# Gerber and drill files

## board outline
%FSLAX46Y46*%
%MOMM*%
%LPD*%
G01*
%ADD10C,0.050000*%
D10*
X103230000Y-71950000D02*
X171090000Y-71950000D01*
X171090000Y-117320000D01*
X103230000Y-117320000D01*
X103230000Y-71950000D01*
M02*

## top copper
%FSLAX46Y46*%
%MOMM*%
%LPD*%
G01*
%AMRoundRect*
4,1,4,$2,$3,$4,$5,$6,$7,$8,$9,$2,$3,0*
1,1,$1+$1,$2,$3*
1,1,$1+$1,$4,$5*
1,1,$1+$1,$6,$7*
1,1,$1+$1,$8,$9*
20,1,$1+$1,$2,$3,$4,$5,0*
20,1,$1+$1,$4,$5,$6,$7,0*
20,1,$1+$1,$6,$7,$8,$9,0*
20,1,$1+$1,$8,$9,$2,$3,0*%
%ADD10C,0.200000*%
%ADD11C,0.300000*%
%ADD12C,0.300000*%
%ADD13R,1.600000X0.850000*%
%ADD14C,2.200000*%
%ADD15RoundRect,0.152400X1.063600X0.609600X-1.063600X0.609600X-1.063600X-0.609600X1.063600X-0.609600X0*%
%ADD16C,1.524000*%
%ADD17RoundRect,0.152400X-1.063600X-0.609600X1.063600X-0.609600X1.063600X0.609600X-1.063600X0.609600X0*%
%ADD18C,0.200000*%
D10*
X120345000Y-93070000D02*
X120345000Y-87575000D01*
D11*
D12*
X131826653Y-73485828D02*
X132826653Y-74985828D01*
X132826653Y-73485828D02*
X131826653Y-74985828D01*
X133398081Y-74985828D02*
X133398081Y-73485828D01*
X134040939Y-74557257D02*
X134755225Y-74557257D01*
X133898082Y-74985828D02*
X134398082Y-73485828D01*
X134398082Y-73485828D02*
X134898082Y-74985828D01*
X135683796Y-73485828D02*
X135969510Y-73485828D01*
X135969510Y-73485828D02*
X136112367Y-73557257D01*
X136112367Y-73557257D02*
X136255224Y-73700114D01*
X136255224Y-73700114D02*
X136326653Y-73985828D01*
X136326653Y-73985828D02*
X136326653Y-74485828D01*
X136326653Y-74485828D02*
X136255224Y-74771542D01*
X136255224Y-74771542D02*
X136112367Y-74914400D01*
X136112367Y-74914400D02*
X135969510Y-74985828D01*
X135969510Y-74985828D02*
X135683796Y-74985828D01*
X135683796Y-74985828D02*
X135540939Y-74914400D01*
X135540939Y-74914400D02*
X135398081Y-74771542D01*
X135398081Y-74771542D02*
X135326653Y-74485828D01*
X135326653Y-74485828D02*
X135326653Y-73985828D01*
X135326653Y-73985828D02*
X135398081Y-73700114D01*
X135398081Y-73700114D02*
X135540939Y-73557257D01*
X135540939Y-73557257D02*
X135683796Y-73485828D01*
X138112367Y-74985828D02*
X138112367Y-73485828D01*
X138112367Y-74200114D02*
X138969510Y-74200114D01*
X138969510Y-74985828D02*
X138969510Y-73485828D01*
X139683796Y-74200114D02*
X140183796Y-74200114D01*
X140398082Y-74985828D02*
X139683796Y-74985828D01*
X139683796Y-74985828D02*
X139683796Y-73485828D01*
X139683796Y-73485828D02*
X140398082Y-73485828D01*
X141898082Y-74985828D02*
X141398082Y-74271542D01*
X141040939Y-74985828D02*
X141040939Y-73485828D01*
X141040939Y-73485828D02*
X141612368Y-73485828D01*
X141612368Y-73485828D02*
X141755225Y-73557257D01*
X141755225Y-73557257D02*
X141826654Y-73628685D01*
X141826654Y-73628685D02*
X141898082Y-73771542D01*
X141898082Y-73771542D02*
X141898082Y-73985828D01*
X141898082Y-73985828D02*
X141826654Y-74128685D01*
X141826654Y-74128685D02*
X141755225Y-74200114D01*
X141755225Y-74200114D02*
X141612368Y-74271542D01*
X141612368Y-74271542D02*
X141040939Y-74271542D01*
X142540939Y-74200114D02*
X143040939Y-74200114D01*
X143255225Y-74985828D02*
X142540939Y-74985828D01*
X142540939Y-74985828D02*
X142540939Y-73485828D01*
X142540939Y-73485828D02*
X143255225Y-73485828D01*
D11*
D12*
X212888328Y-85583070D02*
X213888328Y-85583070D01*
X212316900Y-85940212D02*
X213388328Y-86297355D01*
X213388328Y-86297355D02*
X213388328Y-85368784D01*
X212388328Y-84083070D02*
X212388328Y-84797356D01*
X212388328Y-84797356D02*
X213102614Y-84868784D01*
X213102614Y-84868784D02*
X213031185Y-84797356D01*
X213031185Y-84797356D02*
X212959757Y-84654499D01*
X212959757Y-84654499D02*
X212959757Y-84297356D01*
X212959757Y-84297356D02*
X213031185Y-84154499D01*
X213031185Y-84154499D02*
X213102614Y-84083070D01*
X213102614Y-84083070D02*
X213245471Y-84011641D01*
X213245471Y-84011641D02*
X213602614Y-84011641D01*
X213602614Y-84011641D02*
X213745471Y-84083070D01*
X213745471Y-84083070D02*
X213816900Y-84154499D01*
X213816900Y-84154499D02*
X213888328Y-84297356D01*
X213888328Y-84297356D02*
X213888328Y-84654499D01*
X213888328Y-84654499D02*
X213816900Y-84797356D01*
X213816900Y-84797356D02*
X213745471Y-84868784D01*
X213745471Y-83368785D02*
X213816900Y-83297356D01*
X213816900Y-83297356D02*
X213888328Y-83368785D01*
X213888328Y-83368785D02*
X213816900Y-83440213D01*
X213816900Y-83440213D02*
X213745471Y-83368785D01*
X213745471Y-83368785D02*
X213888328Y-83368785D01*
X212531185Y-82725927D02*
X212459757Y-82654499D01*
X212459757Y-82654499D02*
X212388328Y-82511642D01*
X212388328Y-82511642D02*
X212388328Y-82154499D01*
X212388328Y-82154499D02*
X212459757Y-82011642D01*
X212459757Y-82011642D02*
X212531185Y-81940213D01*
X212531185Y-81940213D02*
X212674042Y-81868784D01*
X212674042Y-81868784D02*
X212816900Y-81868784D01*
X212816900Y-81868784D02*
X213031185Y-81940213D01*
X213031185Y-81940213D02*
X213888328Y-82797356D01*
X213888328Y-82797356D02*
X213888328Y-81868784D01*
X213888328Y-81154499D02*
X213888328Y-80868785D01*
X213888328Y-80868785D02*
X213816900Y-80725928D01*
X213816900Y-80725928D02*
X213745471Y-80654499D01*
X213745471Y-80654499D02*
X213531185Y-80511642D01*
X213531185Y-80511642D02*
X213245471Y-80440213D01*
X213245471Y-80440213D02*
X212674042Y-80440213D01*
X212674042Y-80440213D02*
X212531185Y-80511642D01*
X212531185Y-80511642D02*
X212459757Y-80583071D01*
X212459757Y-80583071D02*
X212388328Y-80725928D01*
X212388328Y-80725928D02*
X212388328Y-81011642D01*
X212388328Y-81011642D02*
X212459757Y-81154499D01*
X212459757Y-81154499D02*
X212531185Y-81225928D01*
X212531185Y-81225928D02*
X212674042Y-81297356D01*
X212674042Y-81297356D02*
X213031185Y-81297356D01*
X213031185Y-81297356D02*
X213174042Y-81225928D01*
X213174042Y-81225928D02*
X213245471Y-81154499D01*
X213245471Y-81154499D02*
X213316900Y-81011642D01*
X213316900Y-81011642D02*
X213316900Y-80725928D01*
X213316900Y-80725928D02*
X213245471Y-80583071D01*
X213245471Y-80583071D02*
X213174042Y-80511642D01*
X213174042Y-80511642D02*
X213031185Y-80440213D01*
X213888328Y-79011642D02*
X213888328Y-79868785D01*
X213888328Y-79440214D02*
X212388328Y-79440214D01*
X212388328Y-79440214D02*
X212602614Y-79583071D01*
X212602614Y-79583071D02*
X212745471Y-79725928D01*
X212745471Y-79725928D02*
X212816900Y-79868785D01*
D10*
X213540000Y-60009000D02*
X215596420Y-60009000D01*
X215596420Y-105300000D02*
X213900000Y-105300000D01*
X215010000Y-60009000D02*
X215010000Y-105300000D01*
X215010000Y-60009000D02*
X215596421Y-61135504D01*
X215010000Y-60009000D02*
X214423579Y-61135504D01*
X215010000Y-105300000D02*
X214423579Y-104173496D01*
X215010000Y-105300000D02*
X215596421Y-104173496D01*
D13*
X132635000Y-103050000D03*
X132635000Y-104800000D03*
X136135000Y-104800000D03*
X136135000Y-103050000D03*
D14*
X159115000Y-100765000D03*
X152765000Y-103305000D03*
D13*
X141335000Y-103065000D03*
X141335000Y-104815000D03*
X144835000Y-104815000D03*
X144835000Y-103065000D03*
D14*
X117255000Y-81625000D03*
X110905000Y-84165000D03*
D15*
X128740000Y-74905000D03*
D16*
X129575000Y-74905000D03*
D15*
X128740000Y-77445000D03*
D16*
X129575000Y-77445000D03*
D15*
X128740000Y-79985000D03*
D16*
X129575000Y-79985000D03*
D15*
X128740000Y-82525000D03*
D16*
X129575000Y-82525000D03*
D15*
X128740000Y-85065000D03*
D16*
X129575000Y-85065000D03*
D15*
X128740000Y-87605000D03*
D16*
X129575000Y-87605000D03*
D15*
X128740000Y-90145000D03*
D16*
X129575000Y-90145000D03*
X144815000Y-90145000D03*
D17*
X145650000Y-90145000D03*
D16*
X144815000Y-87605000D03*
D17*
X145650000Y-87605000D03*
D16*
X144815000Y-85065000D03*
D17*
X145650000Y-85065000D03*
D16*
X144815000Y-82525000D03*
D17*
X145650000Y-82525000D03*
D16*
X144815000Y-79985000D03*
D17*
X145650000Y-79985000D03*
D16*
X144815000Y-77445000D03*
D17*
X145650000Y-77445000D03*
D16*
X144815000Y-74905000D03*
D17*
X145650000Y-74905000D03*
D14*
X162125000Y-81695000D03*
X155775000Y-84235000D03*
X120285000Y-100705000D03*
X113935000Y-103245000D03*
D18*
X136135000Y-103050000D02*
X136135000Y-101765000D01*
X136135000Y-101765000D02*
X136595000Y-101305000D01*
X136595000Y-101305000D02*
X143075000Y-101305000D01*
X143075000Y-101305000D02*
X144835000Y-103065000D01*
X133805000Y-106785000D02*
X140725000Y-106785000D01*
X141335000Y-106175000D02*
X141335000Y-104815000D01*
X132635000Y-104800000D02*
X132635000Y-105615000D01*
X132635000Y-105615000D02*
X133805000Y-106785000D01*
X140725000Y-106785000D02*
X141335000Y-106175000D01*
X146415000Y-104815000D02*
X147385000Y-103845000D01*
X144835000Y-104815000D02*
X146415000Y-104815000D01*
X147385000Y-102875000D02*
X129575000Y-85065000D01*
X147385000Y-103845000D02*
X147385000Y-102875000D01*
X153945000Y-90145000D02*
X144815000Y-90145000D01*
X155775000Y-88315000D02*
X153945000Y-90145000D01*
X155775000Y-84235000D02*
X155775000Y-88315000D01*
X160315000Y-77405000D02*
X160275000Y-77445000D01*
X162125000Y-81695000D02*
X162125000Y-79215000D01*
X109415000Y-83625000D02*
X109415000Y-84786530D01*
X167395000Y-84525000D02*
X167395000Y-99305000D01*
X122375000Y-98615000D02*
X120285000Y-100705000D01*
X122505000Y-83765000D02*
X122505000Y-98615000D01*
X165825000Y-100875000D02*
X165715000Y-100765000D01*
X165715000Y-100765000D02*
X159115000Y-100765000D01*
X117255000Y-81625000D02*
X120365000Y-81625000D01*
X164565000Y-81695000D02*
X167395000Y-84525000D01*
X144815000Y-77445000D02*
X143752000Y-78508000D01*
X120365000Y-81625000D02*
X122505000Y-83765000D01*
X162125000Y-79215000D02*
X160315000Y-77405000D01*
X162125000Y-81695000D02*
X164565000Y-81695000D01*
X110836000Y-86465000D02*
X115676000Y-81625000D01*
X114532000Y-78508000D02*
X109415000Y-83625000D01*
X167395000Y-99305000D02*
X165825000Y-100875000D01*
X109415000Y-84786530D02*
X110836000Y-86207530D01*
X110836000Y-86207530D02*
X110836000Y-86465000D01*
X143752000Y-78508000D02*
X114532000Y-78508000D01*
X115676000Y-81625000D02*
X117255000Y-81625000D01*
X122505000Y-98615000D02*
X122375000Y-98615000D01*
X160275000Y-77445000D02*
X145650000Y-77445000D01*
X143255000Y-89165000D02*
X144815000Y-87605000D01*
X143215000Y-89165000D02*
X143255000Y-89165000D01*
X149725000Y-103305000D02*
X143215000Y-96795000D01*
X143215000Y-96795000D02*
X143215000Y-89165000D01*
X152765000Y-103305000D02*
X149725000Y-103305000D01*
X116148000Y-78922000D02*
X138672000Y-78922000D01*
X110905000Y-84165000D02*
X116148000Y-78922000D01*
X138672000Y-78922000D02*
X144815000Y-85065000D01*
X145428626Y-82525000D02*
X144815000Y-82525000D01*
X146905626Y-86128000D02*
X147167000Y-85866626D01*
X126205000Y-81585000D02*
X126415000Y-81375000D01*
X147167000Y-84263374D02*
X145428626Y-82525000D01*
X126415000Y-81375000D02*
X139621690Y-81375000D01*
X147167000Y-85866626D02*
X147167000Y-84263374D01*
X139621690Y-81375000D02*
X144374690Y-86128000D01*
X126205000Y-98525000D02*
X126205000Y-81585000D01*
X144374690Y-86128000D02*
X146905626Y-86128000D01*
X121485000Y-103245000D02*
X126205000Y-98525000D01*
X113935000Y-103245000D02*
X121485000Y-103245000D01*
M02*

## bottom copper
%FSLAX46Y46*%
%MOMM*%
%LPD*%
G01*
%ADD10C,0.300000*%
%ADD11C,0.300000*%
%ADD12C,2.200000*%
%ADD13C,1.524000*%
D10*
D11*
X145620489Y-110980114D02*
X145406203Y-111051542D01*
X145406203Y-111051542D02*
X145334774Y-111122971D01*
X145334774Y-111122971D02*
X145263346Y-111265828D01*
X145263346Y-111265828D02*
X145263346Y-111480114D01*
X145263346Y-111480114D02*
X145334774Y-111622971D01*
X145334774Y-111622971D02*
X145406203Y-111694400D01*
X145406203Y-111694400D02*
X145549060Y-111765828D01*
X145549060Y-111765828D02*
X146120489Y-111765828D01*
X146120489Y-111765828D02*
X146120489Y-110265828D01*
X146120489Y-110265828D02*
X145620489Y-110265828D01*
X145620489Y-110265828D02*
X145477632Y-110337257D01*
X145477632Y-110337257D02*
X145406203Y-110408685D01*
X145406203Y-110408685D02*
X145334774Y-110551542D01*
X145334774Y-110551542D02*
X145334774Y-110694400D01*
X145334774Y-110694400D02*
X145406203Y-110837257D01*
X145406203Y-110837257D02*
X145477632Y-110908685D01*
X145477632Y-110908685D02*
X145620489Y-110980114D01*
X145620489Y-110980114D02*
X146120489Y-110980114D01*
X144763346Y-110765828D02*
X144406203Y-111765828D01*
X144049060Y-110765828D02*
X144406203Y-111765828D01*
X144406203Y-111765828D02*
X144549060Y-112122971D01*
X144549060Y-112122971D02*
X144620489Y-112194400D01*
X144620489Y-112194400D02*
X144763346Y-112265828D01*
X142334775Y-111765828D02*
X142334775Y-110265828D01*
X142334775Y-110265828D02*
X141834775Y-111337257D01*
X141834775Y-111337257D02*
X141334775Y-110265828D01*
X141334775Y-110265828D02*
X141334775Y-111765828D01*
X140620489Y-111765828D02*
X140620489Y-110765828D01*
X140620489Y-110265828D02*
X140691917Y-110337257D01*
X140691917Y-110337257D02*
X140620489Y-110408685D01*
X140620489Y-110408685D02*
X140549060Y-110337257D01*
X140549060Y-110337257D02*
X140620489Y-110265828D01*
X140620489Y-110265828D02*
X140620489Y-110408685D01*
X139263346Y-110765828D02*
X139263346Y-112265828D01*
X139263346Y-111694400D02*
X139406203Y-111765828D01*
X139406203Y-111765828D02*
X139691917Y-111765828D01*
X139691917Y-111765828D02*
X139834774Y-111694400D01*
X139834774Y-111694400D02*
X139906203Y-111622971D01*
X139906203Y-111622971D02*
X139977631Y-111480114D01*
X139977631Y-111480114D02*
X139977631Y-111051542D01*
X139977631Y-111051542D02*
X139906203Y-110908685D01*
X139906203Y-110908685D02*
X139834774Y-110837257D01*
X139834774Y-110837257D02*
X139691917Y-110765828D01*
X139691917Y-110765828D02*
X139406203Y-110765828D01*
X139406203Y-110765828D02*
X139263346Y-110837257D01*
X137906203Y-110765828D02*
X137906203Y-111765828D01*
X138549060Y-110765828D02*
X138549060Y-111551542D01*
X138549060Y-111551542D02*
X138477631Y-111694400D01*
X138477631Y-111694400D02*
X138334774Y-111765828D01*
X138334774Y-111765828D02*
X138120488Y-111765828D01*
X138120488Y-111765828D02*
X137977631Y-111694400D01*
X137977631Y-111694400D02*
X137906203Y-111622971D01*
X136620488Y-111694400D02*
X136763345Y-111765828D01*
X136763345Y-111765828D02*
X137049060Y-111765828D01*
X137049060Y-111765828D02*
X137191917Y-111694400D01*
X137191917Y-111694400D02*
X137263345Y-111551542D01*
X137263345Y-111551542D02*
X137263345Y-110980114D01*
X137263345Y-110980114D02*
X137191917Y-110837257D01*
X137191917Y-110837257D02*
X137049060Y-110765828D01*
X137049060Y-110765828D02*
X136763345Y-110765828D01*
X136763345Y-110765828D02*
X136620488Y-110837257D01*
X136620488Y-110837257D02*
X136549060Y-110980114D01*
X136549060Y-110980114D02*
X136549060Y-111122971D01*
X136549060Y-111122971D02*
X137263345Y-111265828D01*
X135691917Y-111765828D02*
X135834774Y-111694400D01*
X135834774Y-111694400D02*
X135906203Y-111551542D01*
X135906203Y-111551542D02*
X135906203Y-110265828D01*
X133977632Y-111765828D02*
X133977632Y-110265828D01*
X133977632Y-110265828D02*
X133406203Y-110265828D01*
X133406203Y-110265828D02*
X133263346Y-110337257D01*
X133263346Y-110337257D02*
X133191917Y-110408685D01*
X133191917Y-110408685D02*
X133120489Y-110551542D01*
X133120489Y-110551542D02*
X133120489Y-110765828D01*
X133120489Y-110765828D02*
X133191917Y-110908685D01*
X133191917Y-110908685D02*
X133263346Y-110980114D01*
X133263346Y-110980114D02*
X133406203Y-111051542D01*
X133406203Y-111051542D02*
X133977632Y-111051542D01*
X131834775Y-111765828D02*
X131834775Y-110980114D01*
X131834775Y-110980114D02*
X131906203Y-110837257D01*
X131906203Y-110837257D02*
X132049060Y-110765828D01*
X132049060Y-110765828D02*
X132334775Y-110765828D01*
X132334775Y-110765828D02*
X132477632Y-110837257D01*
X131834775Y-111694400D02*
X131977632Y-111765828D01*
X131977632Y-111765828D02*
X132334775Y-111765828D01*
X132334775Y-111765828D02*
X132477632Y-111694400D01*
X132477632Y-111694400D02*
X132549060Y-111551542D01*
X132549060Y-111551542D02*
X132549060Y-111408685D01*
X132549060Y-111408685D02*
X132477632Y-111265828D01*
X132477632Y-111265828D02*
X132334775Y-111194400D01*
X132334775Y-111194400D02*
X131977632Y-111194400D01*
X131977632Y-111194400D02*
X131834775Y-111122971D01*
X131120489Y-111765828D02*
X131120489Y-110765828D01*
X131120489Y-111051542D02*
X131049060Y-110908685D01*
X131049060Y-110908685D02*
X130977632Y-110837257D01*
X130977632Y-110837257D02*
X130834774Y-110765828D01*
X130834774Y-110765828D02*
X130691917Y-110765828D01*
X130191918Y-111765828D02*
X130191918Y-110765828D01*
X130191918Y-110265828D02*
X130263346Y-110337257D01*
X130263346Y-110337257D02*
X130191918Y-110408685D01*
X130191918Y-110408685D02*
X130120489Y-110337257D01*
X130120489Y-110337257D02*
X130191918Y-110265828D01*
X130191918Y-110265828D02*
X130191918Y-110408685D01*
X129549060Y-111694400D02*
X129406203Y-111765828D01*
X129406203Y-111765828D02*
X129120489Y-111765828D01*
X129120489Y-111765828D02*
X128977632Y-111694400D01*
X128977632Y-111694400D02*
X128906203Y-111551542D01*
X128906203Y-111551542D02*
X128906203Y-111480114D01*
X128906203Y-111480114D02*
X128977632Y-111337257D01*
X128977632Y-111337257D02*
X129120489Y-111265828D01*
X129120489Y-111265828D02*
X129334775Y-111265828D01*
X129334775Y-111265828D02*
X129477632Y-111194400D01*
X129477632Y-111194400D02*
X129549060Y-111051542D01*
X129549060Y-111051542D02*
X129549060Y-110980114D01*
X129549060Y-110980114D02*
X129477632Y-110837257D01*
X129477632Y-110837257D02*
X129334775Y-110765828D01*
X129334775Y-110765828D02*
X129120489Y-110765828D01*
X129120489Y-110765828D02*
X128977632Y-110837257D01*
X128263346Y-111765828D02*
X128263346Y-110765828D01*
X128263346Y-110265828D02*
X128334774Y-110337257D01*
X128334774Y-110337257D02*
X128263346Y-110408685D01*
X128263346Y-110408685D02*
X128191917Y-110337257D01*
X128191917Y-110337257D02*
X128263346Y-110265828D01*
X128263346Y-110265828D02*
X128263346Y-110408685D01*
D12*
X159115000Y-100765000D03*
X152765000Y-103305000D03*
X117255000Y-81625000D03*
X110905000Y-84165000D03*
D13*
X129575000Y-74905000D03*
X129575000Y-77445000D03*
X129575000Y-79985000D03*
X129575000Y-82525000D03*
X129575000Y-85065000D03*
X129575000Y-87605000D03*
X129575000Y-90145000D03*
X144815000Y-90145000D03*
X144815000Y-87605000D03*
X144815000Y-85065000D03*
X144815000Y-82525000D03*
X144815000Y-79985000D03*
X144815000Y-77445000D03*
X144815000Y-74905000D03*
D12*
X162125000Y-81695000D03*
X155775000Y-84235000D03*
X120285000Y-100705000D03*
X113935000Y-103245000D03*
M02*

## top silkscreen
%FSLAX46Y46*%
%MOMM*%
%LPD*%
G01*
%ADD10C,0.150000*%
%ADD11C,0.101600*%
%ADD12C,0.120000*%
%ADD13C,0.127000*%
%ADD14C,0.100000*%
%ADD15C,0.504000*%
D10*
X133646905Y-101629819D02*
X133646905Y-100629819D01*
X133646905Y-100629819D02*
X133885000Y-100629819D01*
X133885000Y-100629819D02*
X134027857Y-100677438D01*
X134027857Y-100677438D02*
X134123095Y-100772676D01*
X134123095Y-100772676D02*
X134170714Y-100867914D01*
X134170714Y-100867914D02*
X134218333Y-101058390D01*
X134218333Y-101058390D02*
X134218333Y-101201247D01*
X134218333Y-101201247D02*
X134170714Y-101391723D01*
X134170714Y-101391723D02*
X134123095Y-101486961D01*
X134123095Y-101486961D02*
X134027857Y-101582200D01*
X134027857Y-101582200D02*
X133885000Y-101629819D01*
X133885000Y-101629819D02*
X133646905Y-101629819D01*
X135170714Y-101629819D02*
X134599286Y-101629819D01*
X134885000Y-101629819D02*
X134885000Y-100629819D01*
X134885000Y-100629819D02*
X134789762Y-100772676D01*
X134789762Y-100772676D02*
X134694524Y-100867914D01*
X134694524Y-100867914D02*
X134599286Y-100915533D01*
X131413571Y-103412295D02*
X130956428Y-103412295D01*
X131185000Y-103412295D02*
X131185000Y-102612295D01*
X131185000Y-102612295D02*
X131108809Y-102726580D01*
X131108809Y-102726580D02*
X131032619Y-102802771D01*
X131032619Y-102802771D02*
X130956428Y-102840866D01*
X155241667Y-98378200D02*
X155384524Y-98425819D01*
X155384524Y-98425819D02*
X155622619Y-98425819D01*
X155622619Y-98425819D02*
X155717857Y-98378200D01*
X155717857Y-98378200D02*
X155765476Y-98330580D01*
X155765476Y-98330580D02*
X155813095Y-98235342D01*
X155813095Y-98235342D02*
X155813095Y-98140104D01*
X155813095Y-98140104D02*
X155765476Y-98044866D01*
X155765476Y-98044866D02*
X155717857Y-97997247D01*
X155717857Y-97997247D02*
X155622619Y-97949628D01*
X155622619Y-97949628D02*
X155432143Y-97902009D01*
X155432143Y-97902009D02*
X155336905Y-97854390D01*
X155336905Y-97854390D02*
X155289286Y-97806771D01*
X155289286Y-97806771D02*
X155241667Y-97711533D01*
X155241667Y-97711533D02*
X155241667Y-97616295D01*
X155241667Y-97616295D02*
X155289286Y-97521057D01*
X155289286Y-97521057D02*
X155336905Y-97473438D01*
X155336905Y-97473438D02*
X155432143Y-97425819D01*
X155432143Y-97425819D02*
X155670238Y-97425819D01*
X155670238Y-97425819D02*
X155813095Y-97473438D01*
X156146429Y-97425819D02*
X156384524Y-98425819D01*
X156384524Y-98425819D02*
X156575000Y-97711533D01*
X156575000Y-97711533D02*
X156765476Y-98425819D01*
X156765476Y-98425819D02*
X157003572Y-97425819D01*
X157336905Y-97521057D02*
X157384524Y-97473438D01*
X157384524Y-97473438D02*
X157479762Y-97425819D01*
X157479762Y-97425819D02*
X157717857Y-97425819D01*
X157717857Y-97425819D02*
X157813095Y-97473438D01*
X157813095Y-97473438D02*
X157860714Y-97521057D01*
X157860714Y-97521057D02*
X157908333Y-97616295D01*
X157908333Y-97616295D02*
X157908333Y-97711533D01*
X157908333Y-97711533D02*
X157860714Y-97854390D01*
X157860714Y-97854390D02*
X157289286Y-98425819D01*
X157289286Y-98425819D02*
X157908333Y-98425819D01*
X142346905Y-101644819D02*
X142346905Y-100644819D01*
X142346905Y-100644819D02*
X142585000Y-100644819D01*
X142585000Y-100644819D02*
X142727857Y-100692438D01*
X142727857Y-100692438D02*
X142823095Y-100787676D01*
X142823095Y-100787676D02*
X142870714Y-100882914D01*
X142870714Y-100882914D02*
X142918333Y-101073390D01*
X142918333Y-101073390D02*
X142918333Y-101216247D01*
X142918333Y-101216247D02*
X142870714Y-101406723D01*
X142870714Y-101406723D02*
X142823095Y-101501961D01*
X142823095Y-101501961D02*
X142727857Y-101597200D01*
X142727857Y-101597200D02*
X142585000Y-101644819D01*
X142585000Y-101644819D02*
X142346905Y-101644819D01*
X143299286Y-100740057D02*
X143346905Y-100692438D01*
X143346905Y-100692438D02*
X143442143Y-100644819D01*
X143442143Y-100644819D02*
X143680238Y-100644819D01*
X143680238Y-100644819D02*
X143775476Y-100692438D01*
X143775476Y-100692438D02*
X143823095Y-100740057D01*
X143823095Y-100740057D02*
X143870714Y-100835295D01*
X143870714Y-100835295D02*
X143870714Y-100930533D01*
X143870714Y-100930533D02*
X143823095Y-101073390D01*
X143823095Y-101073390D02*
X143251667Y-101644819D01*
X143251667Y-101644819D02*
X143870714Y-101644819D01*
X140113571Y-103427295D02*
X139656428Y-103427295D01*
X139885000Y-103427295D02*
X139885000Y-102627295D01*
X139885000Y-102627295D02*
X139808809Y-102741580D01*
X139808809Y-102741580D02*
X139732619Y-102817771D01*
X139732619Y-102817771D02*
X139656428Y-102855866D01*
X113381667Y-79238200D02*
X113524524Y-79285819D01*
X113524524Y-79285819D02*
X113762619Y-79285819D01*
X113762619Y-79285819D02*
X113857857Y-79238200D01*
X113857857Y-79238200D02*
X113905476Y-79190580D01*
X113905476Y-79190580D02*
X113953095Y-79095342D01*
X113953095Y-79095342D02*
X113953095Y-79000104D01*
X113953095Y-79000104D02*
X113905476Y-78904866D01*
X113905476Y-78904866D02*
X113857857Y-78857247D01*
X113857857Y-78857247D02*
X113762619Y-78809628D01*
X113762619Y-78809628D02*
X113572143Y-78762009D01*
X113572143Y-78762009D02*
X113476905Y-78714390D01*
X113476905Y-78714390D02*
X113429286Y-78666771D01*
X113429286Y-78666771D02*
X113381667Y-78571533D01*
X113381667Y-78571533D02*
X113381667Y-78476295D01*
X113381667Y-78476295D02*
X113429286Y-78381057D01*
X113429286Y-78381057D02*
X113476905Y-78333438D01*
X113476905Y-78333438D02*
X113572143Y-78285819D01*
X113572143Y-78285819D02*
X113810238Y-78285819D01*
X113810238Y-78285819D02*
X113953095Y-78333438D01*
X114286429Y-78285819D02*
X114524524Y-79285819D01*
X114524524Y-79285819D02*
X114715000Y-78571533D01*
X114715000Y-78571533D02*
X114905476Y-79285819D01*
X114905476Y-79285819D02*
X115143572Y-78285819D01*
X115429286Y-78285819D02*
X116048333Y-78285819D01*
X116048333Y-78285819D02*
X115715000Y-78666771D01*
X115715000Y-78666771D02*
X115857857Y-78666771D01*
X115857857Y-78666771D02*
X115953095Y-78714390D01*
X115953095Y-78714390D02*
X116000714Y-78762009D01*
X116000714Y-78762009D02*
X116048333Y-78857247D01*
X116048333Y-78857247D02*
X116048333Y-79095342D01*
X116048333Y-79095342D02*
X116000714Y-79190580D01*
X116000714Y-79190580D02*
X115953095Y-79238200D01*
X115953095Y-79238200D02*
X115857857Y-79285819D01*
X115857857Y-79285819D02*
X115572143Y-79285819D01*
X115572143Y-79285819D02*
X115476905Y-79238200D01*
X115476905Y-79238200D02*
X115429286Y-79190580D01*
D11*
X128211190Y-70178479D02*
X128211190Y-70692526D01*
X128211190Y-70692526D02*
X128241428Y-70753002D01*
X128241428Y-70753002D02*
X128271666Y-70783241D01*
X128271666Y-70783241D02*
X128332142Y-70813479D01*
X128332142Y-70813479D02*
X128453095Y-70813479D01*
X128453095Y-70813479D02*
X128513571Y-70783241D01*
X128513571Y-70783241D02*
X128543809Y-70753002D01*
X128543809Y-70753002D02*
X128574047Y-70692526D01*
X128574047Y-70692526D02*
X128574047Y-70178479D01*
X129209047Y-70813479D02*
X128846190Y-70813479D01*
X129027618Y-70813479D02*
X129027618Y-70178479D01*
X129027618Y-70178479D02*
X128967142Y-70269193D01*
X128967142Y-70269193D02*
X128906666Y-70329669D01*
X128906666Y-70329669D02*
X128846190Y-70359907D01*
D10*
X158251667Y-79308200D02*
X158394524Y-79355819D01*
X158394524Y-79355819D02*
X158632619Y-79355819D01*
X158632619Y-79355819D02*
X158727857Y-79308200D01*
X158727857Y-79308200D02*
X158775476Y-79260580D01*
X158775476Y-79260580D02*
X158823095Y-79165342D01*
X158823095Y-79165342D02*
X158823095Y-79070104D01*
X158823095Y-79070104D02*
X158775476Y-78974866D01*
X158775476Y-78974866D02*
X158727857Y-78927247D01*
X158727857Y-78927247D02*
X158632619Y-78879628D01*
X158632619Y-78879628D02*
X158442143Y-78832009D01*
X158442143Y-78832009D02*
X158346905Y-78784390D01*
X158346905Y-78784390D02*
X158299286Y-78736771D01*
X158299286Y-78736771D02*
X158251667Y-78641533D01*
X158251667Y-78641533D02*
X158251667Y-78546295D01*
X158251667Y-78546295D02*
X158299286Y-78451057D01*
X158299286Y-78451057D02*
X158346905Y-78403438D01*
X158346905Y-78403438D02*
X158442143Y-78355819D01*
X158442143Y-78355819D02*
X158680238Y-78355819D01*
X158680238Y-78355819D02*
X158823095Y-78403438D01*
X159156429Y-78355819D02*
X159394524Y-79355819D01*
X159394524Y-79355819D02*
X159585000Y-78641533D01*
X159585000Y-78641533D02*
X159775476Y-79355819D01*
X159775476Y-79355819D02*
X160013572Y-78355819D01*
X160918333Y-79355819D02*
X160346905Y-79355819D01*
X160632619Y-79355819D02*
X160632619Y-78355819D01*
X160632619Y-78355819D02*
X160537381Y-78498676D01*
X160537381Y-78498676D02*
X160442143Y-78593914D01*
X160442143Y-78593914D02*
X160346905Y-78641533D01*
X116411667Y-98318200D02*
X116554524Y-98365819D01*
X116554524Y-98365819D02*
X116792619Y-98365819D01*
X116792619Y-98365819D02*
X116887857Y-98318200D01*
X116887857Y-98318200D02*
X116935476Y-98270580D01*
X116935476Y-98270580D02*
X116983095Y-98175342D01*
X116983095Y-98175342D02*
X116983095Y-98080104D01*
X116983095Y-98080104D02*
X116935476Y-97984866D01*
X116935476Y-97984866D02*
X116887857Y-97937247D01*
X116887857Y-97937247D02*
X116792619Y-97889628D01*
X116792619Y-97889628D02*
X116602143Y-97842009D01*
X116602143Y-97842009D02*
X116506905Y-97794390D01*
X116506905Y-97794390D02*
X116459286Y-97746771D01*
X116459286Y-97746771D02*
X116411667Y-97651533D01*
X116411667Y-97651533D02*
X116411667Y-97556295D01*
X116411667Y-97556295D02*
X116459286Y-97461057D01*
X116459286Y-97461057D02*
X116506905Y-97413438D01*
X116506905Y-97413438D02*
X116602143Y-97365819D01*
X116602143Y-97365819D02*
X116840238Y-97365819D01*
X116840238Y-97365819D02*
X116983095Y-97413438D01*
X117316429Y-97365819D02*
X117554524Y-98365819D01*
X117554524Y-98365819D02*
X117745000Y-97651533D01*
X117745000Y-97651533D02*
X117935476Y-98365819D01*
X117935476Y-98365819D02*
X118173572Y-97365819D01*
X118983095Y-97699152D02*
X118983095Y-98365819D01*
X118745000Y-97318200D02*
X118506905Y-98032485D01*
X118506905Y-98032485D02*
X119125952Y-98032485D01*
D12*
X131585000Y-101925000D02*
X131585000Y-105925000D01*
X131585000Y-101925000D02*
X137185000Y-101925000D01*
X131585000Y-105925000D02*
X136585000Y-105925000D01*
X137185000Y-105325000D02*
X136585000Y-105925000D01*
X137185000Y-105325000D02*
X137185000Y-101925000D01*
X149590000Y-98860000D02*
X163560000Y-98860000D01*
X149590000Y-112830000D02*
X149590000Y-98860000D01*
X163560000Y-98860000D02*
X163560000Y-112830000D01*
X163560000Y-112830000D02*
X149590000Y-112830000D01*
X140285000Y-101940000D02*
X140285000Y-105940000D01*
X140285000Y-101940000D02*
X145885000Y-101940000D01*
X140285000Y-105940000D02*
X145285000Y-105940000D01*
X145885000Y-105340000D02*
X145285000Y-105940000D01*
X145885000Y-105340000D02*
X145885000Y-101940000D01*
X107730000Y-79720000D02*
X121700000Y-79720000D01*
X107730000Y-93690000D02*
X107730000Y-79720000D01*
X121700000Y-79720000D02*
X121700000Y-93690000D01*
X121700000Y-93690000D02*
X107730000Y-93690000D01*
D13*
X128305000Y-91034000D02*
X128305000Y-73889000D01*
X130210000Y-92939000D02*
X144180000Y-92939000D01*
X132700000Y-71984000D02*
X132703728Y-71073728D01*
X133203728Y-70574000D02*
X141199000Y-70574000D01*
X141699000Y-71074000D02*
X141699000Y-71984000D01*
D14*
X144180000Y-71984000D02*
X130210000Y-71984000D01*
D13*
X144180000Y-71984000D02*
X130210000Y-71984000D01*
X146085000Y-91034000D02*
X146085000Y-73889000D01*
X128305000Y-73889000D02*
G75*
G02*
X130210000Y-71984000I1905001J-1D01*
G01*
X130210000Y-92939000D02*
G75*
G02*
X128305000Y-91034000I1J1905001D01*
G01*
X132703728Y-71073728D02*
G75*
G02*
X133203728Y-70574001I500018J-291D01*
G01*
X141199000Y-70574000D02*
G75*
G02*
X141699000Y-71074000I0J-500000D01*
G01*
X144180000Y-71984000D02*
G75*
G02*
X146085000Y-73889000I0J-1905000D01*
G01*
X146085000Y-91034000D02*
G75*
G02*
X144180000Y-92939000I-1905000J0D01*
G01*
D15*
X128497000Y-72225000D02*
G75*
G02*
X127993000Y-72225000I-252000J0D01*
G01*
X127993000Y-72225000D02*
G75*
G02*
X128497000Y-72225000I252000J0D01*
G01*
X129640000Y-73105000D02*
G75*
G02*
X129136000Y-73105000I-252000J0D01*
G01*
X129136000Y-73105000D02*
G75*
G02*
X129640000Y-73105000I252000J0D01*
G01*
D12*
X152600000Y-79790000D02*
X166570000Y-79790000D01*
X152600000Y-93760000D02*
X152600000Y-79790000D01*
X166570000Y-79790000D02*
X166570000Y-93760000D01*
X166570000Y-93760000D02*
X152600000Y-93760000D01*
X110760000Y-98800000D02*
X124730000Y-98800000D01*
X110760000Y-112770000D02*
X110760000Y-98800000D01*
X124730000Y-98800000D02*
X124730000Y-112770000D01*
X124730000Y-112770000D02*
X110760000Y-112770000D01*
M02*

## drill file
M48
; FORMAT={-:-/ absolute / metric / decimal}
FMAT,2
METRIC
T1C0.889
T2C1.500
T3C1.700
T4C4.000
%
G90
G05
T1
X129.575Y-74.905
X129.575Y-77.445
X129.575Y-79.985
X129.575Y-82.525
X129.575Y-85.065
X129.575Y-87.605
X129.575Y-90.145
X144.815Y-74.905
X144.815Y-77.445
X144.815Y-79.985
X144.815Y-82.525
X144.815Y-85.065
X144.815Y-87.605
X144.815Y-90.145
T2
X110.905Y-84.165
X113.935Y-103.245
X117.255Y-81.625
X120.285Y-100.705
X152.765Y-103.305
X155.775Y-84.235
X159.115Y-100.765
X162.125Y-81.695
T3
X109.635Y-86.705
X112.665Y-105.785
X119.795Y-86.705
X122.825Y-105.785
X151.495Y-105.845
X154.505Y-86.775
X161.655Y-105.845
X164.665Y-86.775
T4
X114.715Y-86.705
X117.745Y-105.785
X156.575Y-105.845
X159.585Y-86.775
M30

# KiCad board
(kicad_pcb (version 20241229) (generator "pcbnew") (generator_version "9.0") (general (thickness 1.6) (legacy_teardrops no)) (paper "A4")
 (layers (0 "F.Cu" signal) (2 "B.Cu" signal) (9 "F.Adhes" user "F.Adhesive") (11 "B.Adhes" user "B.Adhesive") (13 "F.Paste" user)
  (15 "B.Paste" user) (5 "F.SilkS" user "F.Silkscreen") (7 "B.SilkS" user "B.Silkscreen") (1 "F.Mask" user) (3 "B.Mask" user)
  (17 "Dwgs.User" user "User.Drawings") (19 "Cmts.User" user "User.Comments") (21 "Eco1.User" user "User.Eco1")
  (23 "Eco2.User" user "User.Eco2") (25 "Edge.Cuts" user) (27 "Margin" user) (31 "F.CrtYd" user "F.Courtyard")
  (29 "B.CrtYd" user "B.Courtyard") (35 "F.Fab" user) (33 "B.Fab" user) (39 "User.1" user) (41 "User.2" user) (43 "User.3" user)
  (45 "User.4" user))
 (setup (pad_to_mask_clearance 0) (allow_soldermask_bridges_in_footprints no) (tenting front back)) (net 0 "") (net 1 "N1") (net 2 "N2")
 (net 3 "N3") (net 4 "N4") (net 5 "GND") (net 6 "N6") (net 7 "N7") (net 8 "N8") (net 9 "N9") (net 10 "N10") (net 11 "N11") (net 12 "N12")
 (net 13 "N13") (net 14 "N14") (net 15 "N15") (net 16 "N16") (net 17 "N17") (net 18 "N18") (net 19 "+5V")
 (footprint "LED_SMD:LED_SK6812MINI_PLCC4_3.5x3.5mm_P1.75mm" (layer "F.Cu") (at 134.385 103.925)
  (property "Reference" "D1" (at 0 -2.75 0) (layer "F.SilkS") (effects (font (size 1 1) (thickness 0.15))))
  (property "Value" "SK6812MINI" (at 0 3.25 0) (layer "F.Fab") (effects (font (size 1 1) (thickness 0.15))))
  (fp_line (start -2.8 -2) (end -2.8 2) (stroke (width 0.12) (type default)) (layer "F.SilkS"))
  (fp_line (start -2.8 -2) (end 2.8 -2) (stroke (width 0.12) (type solid)) (layer "F.SilkS"))
  (fp_line (start -2.8 2) (end 2.2 2) (stroke (width 0.12) (type solid)) (layer "F.SilkS"))
  (fp_line (start 2.8 1.4) (end 2.2 2) (stroke (width 0.12) (type default)) (layer "F.SilkS"))
  (fp_line (start 2.8 1.4) (end 2.8 -2) (stroke (width 0.12) (type solid)) (layer "F.SilkS"))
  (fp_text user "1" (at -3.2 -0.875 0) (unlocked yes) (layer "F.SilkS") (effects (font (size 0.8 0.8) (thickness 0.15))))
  (pad "1" smd rect (at -1.75 -0.875) (size 1.6 0.85) (layers "F.Cu" "F.Mask" "F.Paste") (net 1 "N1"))
  (pad "2" smd rect (at -1.75 0.875) (size 1.6 0.85) (layers "F.Cu" "F.Mask" "F.Paste") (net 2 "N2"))
  (pad "3" smd rect (at 1.75 0.875) (size 1.6 0.85) (layers "F.Cu" "F.Mask" "F.Paste") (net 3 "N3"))
  (pad "4" smd rect (at 1.75 -0.875) (size 1.6 0.85) (layers "F.Cu" "F.Mask" "F.Paste") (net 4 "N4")))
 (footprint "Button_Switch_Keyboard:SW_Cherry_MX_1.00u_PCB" (layer "F.Cu") (at 159.115 100.765)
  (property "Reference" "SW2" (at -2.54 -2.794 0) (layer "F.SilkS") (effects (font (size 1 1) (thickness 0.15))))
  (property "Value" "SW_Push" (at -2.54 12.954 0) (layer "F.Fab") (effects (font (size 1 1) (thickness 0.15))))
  (fp_line (start -9.525 -1.905) (end 4.445 -1.905) (stroke (width 0.12) (type solid)) (layer "F.SilkS"))
  (fp_line (start -9.525 12.065) (end -9.525 -1.905) (stroke (width 0.12) (type solid)) (layer "F.SilkS"))
  (fp_line (start 4.445 -1.905) (end 4.445 12.065) (stroke (width 0.12) (type solid)) (layer "F.SilkS"))
  (fp_line (start 4.445 12.065) (end -9.525 12.065) (stroke (width 0.12) (type solid)) (layer "F.SilkS"))
  (pad "" np_thru_hole circle (at -7.62 5.08) (size 1.7 1.7) (drill 1.7) (layers "*.Cu" "*.Mask"))
  (pad "" np_thru_hole circle (at -2.54 5.08) (size 4 4) (drill 4) (layers "*.Cu" "*.Mask"))
  (pad "" np_thru_hole circle (at 2.54 5.08) (size 1.7 1.7) (drill 1.7) (layers "*.Cu" "*.Mask"))
  (pad "1" thru_hole circle (at 0 0) (size 2.2 2.2) (drill 1.5) (layers "*.Cu" "*.Mask") (remove_unused_layers no) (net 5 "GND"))
  (pad "2" thru_hole circle (at -6.35 2.54) (size 2.2 2.2) (drill 1.5) (layers "*.Cu" "*.Mask") (remove_unused_layers no) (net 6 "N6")))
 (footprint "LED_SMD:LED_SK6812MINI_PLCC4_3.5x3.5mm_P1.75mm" (layer "F.Cu") (at 143.085 103.94)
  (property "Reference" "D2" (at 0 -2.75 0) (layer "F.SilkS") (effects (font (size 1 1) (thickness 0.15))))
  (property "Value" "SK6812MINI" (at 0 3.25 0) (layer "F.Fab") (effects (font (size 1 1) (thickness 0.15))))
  (fp_line (start -2.8 -2) (end -2.8 2) (stroke (width 0.12) (type default)) (layer "F.SilkS"))
  (fp_line (start -2.8 -2) (end 2.8 -2) (stroke (width 0.12) (type solid)) (layer "F.SilkS"))
  (fp_line (start -2.8 2) (end 2.2 2) (stroke (width 0.12) (type solid)) (layer "F.SilkS"))
  (fp_line (start 2.8 1.4) (end 2.2 2) (stroke (width 0.12) (type default)) (layer "F.SilkS"))
  (fp_line (start 2.8 1.4) (end 2.8 -2) (stroke (width 0.12) (type solid)) (layer "F.SilkS"))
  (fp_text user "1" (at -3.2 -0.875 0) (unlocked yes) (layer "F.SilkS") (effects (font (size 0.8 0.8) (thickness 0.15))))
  (pad "1" smd rect (at -1.75 -0.875) (size 1.6 0.85) (layers "F.Cu" "F.Mask" "F.Paste") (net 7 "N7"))
  (pad "2" smd rect (at -1.75 0.875) (size 1.6 0.85) (layers "F.Cu" "F.Mask" "F.Paste") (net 2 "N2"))
  (pad "3" smd rect (at 1.75 0.875) (size 1.6 0.85) (layers "F.Cu" "F.Mask" "F.Paste") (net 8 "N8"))
  (pad "4" smd rect (at 1.75 -0.875) (size 1.6 0.85) (layers "F.Cu" "F.Mask" "F.Paste") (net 4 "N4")))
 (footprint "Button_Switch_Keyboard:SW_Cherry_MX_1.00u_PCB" (layer "F.Cu") (at 117.255 81.625)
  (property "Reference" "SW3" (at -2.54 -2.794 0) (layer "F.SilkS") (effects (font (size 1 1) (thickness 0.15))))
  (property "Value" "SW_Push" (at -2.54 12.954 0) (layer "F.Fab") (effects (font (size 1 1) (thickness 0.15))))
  (fp_line (start -9.525 -1.905) (end 4.445 -1.905) (stroke (width 0.12) (type solid)) (layer "F.SilkS"))
  (fp_line (start -9.525 12.065) (end -9.525 -1.905) (stroke (width 0.12) (type solid)) (layer "F.SilkS"))
  (fp_line (start 4.445 -1.905) (end 4.445 12.065) (stroke (width 0.12) (type solid)) (layer "F.SilkS"))
  (fp_line (start 4.445 12.065) (end -9.525 12.065) (stroke (width 0.12) (type solid)) (layer "F.SilkS"))
  (pad "" np_thru_hole circle (at -7.62 5.08) (size 1.7 1.7) (drill 1.7) (layers "*.Cu" "*.Mask"))
  (pad "" np_thru_hole circle (at -2.54 5.08) (size 4 4) (drill 4) (layers "*.Cu" "*.Mask"))
  (pad "" np_thru_hole circle (at 2.54 5.08) (size 1.7 1.7) (drill 1.7) (layers "*.Cu" "*.Mask"))
  (pad "1" thru_hole circle (at 0 0) (size 2.2 2.2) (drill 1.5) (layers "*.Cu" "*.Mask") (remove_unused_layers no) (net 5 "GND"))
  (pad "2" thru_hole circle (at -6.35 2.54) (size 2.2 2.2) (drill 1.5) (layers "*.Cu" "*.Mask") (remove_unused_layers no) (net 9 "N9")))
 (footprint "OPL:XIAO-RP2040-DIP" (layer "F.Cu") (at 137.195 82.525)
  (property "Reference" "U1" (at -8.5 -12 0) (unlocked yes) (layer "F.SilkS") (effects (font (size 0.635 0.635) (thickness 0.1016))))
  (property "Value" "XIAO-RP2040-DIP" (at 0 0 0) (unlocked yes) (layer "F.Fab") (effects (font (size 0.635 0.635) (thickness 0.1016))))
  (fp_line (start -8.89 8.509) (end -8.89 -8.636) (stroke (width 0.127) (type solid)) (layer "F.SilkS"))
  (fp_line (start -6.985 10.414) (end 6.985 10.414) (stroke (width 0.127) (type solid)) (layer "F.SilkS"))
  (fp_line (start -4.495 -10.541) (end -4.491272 -11.451272) (stroke (width 0.127) (type solid)) (layer "F.SilkS"))
  (fp_line (start -3.991272 -11.951) (end 4.004 -11.951) (stroke (width 0.127) (type solid)) (layer "F.SilkS"))
  (fp_line (start 4.504 -11.451) (end 4.504 -10.541) (stroke (width 0.127) (type solid)) (layer "F.SilkS"))
  (fp_line (start 6.985 -10.541) (end -6.985 -10.541) (stroke (width 0.1) (type solid)) (layer "F.SilkS"))
  (fp_line (start 6.985 -10.541) (end -6.985 -10.541) (stroke (width 0.127) (type solid)) (layer "F.SilkS"))
  (fp_line (start 8.89 8.509) (end 8.89 -8.636) (stroke (width 0.127) (type solid)) (layer "F.SilkS"))
  (fp_arc (start -8.89 -8.636) (mid -8.332038 -9.983038) (end -6.985 -10.541) (stroke (width 0.127) (type solid)) (layer "F.SilkS"))
  (fp_arc (start -6.985 10.414) (mid -8.332038 9.856038) (end -8.89 8.509) (stroke (width 0.127) (type solid)) (layer "F.SilkS"))
  (fp_arc (start -4.491272 -11.451272) (mid -4.344728 -11.80464) (end -3.991272 -11.951) (stroke (width 0.127) (type default))
   (layer "F.SilkS"))
  (fp_arc (start 4.004 -11.951) (mid 4.357553 -11.804553) (end 4.504 -11.451) (stroke (width 0.127) (type default)) (layer "F.SilkS"))
  (fp_arc (start 6.985 -10.541) (mid 8.332038 -9.983038) (end 8.89 -8.636) (stroke (width 0.127) (type solid)) (layer "F.SilkS"))
  (fp_arc (start 8.89 8.509) (mid 8.332038 9.856038) (end 6.985 10.414) (stroke (width 0.127) (type solid)) (layer "F.SilkS"))
  (fp_circle (center -8.95 -10.3) (end -8.95 -10.554) (stroke (width 0.5) (type solid)) (fill yes) (layer "F.SilkS"))
  (fp_circle (center -7.807 -9.42) (end -7.807 -9.674) (stroke (width 0.5) (type solid)) (fill yes) (layer "F.SilkS"))
  (pad "1" smd roundrect (at -8.455 -7.62 180) (size 2.432 1.524) (layers "F.Cu" "F.Mask") (roundrect_rratio 0.1) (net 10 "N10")
   (thermal_bridge_angle 45))
  (pad "1" thru_hole circle (at -7.62 -7.62 180) (size 1.524 1.524) (drill 0.889) (layers "*.Cu" "*.Mask") (remove_unused_layers no)
   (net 10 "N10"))
  (pad "2" smd roundrect (at -8.455 -5.08 180) (size 2.432 1.524) (layers "F.Cu" "F.Mask") (roundrect_rratio 0.1) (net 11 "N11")
   (thermal_bridge_angle 45))
  (pad "2" thru_hole circle (at -7.62 -5.08 180) (size 1.524 1.524) (drill 0.889) (layers "*.Cu" "*.Mask") (remove_unused_layers no)
   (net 11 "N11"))
  (pad "3" smd roundrect (at -8.455 -2.54 180) (size 2.432 1.524) (layers "F.Cu" "F.Mask") (roundrect_rratio 0.1) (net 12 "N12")
   (thermal_bridge_angle 45))
  (pad "3" thru_hole circle (at -7.62 -2.54 180) (size 1.524 1.524) (drill 0.889) (layers "*.Cu" "*.Mask") (remove_unused_layers no)
   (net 12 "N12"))
  (pad "4" smd roundrect (at -8.455 0 180) (size 2.432 1.524) (layers "F.Cu" "F.Mask") (roundrect_rratio 0.1) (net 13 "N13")
   (thermal_bridge_angle 45))
  (pad "4" thru_hole circle (at -7.62 0 180) (size 1.524 1.524) (drill 0.889) (layers "*.Cu" "*.Mask") (remove_unused_layers no)
   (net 13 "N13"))
  (pad "5" smd roundrect (at -8.455 2.54 180) (size 2.432 1.524) (layers "F.Cu" "F.Mask") (roundrect_rratio 0.1) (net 8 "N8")
   (thermal_bridge_angle 45))
  (pad "5" thru_hole circle (at -7.62 2.54 180) (size 1.524 1.524) (drill 0.889) (layers "*.Cu" "*.Mask") (remove_unused_layers no)
   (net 8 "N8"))
  (pad "6" smd roundrect (at -8.455 5.08 180) (size 2.432 1.524) (layers "F.Cu" "F.Mask") (roundrect_rratio 0.1) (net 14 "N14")
   (thermal_bridge_angle 45))
  (pad "6" thru_hole circle (at -7.62 5.08 180) (size 1.524 1.524) (drill 0.889) (layers "*.Cu" "*.Mask") (remove_unused_layers no)
   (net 14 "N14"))
  (pad "7" smd roundrect (at -8.455 7.62 180) (size 2.432 1.524) (layers "F.Cu" "F.Mask") (roundrect_rratio 0.1) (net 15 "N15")
   (thermal_bridge_angle 45))
  (pad "7" thru_hole circle (at -7.62 7.62 180) (size 1.524 1.524) (drill 0.889) (layers "*.Cu" "*.Mask") (remove_unused_layers no)
   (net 15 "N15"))
  (pad "8" thru_hole circle (at 7.62 7.62) (size 1.524 1.524) (drill 0.889) (layers "*.Cu" "*.Mask") (remove_unused_layers no)
   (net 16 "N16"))
  (pad "8" smd roundrect (at 8.455 7.62) (size 2.432 1.524) (layers "F.Cu" "F.Mask") (roundrect_rratio 0.1) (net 16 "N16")
   (thermal_bridge_angle 45))
  (pad "9" thru_hole circle (at 7.62 5.08) (size 1.524 1.524) (drill 0.889) (layers "*.Cu" "*.Mask") (remove_unused_layers no) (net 6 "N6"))
  (pad "9" smd roundrect (at 8.455 5.08) (size 2.432 1.524) (layers "F.Cu" "F.Mask") (roundrect_rratio 0.1) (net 6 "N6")
   (thermal_bridge_angle 45))
  (pad "10" thru_hole circle (at 7.62 2.54) (size 1.524 1.524) (drill 0.889) (layers "*.Cu" "*.Mask") (remove_unused_layers no) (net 9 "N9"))
  (pad "10" smd roundrect (at 8.455 2.54) (size 2.432 1.524) (layers "F.Cu" "F.Mask") (roundrect_rratio 0.1) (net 9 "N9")
   (thermal_bridge_angle 45))
  (pad "11" thru_hole circle (at 7.62 0) (size 1.524 1.524) (drill 0.889) (layers "*.Cu" "*.Mask") (remove_unused_layers no) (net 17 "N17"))
  (pad "11" smd roundrect (at 8.455 0) (size 2.432 1.524) (layers "F.Cu" "F.Mask") (roundrect_rratio 0.1) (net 17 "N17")
   (thermal_bridge_angle 45))
  (pad "12" thru_hole circle (at 7.62 -2.54) (size 1.524 1.524) (drill 0.889) (layers "*.Cu" "*.Mask") (remove_unused_layers no)
   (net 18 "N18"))
  (pad "12" smd roundrect (at 8.455 -2.54) (size 2.432 1.524) (layers "F.Cu" "F.Mask") (roundrect_rratio 0.1) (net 18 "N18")
   (thermal_bridge_angle 45))
  (pad "13" thru_hole circle (at 7.62 -5.08) (size 1.524 1.524) (drill 0.889) (layers "*.Cu" "*.Mask") (remove_unused_layers no)
   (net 5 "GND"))
  (pad "13" smd roundrect (at 8.455 -5.08) (size 2.432 1.524) (layers "F.Cu" "F.Mask") (roundrect_rratio 0.1) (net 5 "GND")
   (thermal_bridge_angle 45))
  (pad "14" thru_hole circle (at 7.62 -7.62) (size 1.524 1.524) (drill 0.889) (layers "*.Cu" "*.Mask") (remove_unused_layers no)
   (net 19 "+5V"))
  (pad "14" smd roundrect (at 8.455 -7.62) (size 2.432 1.524) (layers "F.Cu" "F.Mask") (roundrect_rratio 0.1) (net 19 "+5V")
   (thermal_bridge_angle 45)))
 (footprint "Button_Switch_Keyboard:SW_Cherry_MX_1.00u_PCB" (layer "F.Cu") (at 162.125 81.695)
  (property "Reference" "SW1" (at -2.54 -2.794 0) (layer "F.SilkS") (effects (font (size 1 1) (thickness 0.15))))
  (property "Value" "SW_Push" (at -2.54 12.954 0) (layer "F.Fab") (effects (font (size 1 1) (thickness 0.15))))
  (fp_line (start -9.525 -1.905) (end 4.445 -1.905) (stroke (width 0.12) (type solid)) (layer "F.SilkS"))
  (fp_line (start -9.525 12.065) (end -9.525 -1.905) (stroke (width 0.12) (type solid)) (layer "F.SilkS"))
  (fp_line (start 4.445 -1.905) (end 4.445 12.065) (stroke (width 0.12) (type solid)) (layer "F.SilkS"))
  (fp_line (start 4.445 12.065) (end -9.525 12.065) (stroke (width 0.12) (type solid)) (layer "F.SilkS"))
  (pad "" np_thru_hole circle (at -7.62 5.08) (size 1.7 1.7) (drill 1.7) (layers "*.Cu" "*.Mask"))
  (pad "" np_thru_hole circle (at -2.54 5.08) (size 4 4) (drill 4) (layers "*.Cu" "*.Mask"))
  (pad "" np_thru_hole circle (at 2.54 5.08) (size 1.7 1.7) (drill 1.7) (layers "*.Cu" "*.Mask"))
  (pad "1" thru_hole circle (at 0 0) (size 2.2 2.2) (drill 1.5) (layers "*.Cu" "*.Mask") (remove_unused_layers no) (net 5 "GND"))
  (pad "2" thru_hole circle (at -6.35 2.54) (size 2.2 2.2) (drill 1.5) (layers "*.Cu" "*.Mask") (remove_unused_layers no) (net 16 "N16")))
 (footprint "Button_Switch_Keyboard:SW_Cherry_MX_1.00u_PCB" (layer "F.Cu") (at 120.285 100.705)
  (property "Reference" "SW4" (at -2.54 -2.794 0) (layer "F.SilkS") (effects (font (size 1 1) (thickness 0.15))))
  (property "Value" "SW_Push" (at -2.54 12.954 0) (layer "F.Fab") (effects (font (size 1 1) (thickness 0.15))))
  (fp_line (start -9.525 -1.905) (end 4.445 -1.905) (stroke (width 0.12) (type solid)) (layer "F.SilkS"))
  (fp_line (start -9.525 12.065) (end -9.525 -1.905) (stroke (width 0.12) (type solid)) (layer "F.SilkS"))
  (fp_line (start 4.445 -1.905) (end 4.445 12.065) (stroke (width 0.12) (type solid)) (layer "F.SilkS"))
  (fp_line (start 4.445 12.065) (end -9.525 12.065) (stroke (width 0.12) (type solid)) (layer "F.SilkS"))
  (pad "" np_thru_hole circle (at -7.62 5.08) (size 1.7 1.7) (drill 1.7) (layers "*.Cu" "*.Mask"))
  (pad "" np_thru_hole circle (at -2.54 5.08) (size 4 4) (drill 4) (layers "*.Cu" "*.Mask"))
  (pad "" np_thru_hole circle (at 2.54 5.08) (size 1.7 1.7) (drill 1.7) (layers "*.Cu" "*.Mask"))
  (pad "1" thru_hole circle (at 0 0) (size 2.2 2.2) (drill 1.5) (layers "*.Cu" "*.Mask") (remove_unused_layers no) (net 5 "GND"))
  (pad "2" thru_hole circle (at -6.35 2.54) (size 2.2 2.2) (drill 1.5) (layers "*.Cu" "*.Mask") (remove_unused_layers no) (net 17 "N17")))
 (gr_line (start 120.345 93.07) (end 120.345 87.575) (stroke (width 0.2) (type default)) (layer "F.Cu"))
 (gr_rect (start 103.23 71.95) (end 171.09 117.32) (stroke (width 0.05) (type default)) (fill no) (layer "Edge.Cuts"))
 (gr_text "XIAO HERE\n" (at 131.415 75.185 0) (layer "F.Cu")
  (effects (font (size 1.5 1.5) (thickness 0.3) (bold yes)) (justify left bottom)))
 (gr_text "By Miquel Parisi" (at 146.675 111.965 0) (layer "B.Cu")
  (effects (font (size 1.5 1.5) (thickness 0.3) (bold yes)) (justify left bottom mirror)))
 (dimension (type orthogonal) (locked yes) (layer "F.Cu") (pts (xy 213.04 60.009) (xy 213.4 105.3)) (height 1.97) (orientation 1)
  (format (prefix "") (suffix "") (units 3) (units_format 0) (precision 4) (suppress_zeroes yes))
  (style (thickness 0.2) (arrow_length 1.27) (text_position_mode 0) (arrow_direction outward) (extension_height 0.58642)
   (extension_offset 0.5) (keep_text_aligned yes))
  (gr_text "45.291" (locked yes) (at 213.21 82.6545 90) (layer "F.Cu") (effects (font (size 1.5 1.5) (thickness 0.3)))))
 (segment (start 136.135 103.05) (end 136.135 101.765) (width 0.2) (layer "F.Cu") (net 4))
 (segment (start 136.135 101.765) (end 136.595 101.305) (width 0.2) (layer "F.Cu") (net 4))
 (segment (start 136.595 101.305) (end 143.075 101.305) (width 0.2) (layer "F.Cu") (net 4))
 (segment (start 143.075 101.305) (end 144.835 103.065) (width 0.2) (layer "F.Cu") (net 4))
 (segment (start 133.805 106.785) (end 140.725 106.785) (width 0.2) (layer "F.Cu") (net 2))
 (segment (start 141.335 106.175) (end 141.335 104.815) (width 0.2) (layer "F.Cu") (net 2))
 (segment (start 132.635 104.8) (end 132.635 105.615) (width 0.2) (layer "F.Cu") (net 2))
 (segment (start 132.635 105.615) (end 133.805 106.785) (width 0.2) (layer "F.Cu") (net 2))
 (segment (start 140.725 106.785) (end 141.335 106.175) (width 0.2) (layer "F.Cu") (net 2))
 (segment (start 146.415 104.815) (end 147.385 103.845) (width 0.2) (layer "F.Cu") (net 8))
 (segment (start 144.835 104.815) (end 146.415 104.815) (width 0.2) (layer "F.Cu") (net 8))
 (segment (start 147.385 102.875) (end 129.575 85.065) (width 0.2) (layer "F.Cu") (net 8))
 (segment (start 147.385 103.845) (end 147.385 102.875) (width 0.2) (layer "F.Cu") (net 8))
 (segment (start 153.945 90.145) (end 144.815 90.145) (width 0.2) (layer "F.Cu") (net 16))
 (segment (start 155.775 88.315) (end 153.945 90.145) (width 0.2) (layer "F.Cu") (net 16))
 (segment (start 155.775 84.235) (end 155.775 88.315) (width 0.2) (layer "F.Cu") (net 16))
 (segment (start 160.315 77.405) (end 160.275 77.445) (width 0.2) (layer "F.Cu") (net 5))
 (segment (start 162.125 81.695) (end 162.125 79.215) (width 0.2) (layer "F.Cu") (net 5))
 (segment (start 109.415 83.625) (end 109.415 84.78653) (width 0.2) (layer "F.Cu") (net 5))
 (segment (start 167.395 84.525) (end 167.395 99.305) (width 0.2) (layer "F.Cu") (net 5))
 (segment (start 122.375 98.615) (end 120.285 100.705) (width 0.2) (layer "F.Cu") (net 5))
 (segment (start 122.505 83.765) (end 122.505 98.615) (width 0.2) (layer "F.Cu") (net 5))
 (segment (start 165.825 100.875) (end 165.715 100.765) (width 0.2) (layer "F.Cu") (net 5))
 (segment (start 165.715 100.765) (end 159.115 100.765) (width 0.2) (layer "F.Cu") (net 5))
 (segment (start 117.255 81.625) (end 120.365 81.625) (width 0.2) (layer "F.Cu") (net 5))
 (segment (start 164.565 81.695) (end 167.395 84.525) (width 0.2) (layer "F.Cu") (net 5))
 (segment (start 144.815 77.445) (end 143.752 78.508) (width 0.2) (layer "F.Cu") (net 5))
 (segment (start 120.365 81.625) (end 122.505 83.765) (width 0.2) (layer "F.Cu") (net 5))
 (segment (start 162.125 79.215) (end 160.315 77.405) (width 0.2) (layer "F.Cu") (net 5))
 (segment (start 162.125 81.695) (end 164.565 81.695) (width 0.2) (layer "F.Cu") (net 5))
 (segment (start 110.836 86.465) (end 115.676 81.625) (width 0.2) (layer "F.Cu") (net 5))
 (segment (start 114.532 78.508) (end 109.415 83.625) (width 0.2) (layer "F.Cu") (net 5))
 (segment (start 167.395 99.305) (end 165.825 100.875) (width 0.2) (layer "F.Cu") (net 5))
 (segment (start 109.415 84.78653) (end 110.836 86.20753) (width 0.2) (layer "F.Cu") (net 5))
 (segment (start 110.836 86.20753) (end 110.836 86.465) (width 0.2) (layer "F.Cu") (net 5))
 (segment (start 143.752 78.508) (end 114.532 78.508) (width 0.2) (layer "F.Cu") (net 5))
 (segment (start 115.676 81.625) (end 117.255 81.625) (width 0.2) (layer "F.Cu") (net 5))
 (segment (start 122.505 98.615) (end 122.375 98.615) (width 0.2) (layer "F.Cu") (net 5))
 (segment (start 160.275 77.445) (end 145.65 77.445) (width 0.2) (layer "F.Cu") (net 5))
 (segment (start 143.255 89.165) (end 144.815 87.605) (width 0.2) (layer "F.Cu") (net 6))
 (segment (start 143.215 89.165) (end 143.255 89.165) (width 0.2) (layer "F.Cu") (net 6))
 (segment (start 149.725 103.305) (end 143.215 96.795) (width 0.2) (layer "F.Cu") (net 6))
 (segment (start 143.215 96.795) (end 143.215 89.165) (width 0.2) (layer "F.Cu") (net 6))
 (segment (start 152.765 103.305) (end 149.725 103.305) (width 0.2) (layer "F.Cu") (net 6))
 (segment (start 116.148 78.922) (end 138.672 78.922) (width 0.2) (layer "F.Cu") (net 9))
 (segment (start 110.905 84.165) (end 116.148 78.922) (width 0.2) (layer "F.Cu") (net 9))
 (segment (start 138.672 78.922) (end 144.815 85.065) (width 0.2) (layer "F.Cu") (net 9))
 (segment (start 145.428626 82.525) (end 144.815 82.525) (width 0.2) (layer "F.Cu") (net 17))
 (segment (start 146.905626 86.128) (end 147.167 85.866626) (width 0.2) (layer "F.Cu") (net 17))
 (segment (start 126.205 81.585) (end 126.415 81.375) (width 0.2) (layer "F.Cu") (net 17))
 (segment (start 147.167 84.263374) (end 145.428626 82.525) (width 0.2) (layer "F.Cu") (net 17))
 (segment (start 126.415 81.375) (end 139.62169 81.375) (width 0.2) (layer "F.Cu") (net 17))
 (segment (start 147.167 85.866626) (end 147.167 84.263374) (width 0.2) (layer "F.Cu") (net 17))
 (segment (start 139.62169 81.375) (end 144.37469 86.128) (width 0.2) (layer "F.Cu") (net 17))
 (segment (start 126.205 98.525) (end 126.205 81.585) (width 0.2) (layer "F.Cu") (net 17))
 (segment (start 144.37469 86.128) (end 146.905626 86.128) (width 0.2) (layer "F.Cu") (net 17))
 (segment (start 121.485 103.245) (end 126.205 98.525) (width 0.2) (layer "F.Cu") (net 17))
 (segment (start 113.935 103.245) (end 121.485 103.245) (width 0.2) (layer "F.Cu") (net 17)))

